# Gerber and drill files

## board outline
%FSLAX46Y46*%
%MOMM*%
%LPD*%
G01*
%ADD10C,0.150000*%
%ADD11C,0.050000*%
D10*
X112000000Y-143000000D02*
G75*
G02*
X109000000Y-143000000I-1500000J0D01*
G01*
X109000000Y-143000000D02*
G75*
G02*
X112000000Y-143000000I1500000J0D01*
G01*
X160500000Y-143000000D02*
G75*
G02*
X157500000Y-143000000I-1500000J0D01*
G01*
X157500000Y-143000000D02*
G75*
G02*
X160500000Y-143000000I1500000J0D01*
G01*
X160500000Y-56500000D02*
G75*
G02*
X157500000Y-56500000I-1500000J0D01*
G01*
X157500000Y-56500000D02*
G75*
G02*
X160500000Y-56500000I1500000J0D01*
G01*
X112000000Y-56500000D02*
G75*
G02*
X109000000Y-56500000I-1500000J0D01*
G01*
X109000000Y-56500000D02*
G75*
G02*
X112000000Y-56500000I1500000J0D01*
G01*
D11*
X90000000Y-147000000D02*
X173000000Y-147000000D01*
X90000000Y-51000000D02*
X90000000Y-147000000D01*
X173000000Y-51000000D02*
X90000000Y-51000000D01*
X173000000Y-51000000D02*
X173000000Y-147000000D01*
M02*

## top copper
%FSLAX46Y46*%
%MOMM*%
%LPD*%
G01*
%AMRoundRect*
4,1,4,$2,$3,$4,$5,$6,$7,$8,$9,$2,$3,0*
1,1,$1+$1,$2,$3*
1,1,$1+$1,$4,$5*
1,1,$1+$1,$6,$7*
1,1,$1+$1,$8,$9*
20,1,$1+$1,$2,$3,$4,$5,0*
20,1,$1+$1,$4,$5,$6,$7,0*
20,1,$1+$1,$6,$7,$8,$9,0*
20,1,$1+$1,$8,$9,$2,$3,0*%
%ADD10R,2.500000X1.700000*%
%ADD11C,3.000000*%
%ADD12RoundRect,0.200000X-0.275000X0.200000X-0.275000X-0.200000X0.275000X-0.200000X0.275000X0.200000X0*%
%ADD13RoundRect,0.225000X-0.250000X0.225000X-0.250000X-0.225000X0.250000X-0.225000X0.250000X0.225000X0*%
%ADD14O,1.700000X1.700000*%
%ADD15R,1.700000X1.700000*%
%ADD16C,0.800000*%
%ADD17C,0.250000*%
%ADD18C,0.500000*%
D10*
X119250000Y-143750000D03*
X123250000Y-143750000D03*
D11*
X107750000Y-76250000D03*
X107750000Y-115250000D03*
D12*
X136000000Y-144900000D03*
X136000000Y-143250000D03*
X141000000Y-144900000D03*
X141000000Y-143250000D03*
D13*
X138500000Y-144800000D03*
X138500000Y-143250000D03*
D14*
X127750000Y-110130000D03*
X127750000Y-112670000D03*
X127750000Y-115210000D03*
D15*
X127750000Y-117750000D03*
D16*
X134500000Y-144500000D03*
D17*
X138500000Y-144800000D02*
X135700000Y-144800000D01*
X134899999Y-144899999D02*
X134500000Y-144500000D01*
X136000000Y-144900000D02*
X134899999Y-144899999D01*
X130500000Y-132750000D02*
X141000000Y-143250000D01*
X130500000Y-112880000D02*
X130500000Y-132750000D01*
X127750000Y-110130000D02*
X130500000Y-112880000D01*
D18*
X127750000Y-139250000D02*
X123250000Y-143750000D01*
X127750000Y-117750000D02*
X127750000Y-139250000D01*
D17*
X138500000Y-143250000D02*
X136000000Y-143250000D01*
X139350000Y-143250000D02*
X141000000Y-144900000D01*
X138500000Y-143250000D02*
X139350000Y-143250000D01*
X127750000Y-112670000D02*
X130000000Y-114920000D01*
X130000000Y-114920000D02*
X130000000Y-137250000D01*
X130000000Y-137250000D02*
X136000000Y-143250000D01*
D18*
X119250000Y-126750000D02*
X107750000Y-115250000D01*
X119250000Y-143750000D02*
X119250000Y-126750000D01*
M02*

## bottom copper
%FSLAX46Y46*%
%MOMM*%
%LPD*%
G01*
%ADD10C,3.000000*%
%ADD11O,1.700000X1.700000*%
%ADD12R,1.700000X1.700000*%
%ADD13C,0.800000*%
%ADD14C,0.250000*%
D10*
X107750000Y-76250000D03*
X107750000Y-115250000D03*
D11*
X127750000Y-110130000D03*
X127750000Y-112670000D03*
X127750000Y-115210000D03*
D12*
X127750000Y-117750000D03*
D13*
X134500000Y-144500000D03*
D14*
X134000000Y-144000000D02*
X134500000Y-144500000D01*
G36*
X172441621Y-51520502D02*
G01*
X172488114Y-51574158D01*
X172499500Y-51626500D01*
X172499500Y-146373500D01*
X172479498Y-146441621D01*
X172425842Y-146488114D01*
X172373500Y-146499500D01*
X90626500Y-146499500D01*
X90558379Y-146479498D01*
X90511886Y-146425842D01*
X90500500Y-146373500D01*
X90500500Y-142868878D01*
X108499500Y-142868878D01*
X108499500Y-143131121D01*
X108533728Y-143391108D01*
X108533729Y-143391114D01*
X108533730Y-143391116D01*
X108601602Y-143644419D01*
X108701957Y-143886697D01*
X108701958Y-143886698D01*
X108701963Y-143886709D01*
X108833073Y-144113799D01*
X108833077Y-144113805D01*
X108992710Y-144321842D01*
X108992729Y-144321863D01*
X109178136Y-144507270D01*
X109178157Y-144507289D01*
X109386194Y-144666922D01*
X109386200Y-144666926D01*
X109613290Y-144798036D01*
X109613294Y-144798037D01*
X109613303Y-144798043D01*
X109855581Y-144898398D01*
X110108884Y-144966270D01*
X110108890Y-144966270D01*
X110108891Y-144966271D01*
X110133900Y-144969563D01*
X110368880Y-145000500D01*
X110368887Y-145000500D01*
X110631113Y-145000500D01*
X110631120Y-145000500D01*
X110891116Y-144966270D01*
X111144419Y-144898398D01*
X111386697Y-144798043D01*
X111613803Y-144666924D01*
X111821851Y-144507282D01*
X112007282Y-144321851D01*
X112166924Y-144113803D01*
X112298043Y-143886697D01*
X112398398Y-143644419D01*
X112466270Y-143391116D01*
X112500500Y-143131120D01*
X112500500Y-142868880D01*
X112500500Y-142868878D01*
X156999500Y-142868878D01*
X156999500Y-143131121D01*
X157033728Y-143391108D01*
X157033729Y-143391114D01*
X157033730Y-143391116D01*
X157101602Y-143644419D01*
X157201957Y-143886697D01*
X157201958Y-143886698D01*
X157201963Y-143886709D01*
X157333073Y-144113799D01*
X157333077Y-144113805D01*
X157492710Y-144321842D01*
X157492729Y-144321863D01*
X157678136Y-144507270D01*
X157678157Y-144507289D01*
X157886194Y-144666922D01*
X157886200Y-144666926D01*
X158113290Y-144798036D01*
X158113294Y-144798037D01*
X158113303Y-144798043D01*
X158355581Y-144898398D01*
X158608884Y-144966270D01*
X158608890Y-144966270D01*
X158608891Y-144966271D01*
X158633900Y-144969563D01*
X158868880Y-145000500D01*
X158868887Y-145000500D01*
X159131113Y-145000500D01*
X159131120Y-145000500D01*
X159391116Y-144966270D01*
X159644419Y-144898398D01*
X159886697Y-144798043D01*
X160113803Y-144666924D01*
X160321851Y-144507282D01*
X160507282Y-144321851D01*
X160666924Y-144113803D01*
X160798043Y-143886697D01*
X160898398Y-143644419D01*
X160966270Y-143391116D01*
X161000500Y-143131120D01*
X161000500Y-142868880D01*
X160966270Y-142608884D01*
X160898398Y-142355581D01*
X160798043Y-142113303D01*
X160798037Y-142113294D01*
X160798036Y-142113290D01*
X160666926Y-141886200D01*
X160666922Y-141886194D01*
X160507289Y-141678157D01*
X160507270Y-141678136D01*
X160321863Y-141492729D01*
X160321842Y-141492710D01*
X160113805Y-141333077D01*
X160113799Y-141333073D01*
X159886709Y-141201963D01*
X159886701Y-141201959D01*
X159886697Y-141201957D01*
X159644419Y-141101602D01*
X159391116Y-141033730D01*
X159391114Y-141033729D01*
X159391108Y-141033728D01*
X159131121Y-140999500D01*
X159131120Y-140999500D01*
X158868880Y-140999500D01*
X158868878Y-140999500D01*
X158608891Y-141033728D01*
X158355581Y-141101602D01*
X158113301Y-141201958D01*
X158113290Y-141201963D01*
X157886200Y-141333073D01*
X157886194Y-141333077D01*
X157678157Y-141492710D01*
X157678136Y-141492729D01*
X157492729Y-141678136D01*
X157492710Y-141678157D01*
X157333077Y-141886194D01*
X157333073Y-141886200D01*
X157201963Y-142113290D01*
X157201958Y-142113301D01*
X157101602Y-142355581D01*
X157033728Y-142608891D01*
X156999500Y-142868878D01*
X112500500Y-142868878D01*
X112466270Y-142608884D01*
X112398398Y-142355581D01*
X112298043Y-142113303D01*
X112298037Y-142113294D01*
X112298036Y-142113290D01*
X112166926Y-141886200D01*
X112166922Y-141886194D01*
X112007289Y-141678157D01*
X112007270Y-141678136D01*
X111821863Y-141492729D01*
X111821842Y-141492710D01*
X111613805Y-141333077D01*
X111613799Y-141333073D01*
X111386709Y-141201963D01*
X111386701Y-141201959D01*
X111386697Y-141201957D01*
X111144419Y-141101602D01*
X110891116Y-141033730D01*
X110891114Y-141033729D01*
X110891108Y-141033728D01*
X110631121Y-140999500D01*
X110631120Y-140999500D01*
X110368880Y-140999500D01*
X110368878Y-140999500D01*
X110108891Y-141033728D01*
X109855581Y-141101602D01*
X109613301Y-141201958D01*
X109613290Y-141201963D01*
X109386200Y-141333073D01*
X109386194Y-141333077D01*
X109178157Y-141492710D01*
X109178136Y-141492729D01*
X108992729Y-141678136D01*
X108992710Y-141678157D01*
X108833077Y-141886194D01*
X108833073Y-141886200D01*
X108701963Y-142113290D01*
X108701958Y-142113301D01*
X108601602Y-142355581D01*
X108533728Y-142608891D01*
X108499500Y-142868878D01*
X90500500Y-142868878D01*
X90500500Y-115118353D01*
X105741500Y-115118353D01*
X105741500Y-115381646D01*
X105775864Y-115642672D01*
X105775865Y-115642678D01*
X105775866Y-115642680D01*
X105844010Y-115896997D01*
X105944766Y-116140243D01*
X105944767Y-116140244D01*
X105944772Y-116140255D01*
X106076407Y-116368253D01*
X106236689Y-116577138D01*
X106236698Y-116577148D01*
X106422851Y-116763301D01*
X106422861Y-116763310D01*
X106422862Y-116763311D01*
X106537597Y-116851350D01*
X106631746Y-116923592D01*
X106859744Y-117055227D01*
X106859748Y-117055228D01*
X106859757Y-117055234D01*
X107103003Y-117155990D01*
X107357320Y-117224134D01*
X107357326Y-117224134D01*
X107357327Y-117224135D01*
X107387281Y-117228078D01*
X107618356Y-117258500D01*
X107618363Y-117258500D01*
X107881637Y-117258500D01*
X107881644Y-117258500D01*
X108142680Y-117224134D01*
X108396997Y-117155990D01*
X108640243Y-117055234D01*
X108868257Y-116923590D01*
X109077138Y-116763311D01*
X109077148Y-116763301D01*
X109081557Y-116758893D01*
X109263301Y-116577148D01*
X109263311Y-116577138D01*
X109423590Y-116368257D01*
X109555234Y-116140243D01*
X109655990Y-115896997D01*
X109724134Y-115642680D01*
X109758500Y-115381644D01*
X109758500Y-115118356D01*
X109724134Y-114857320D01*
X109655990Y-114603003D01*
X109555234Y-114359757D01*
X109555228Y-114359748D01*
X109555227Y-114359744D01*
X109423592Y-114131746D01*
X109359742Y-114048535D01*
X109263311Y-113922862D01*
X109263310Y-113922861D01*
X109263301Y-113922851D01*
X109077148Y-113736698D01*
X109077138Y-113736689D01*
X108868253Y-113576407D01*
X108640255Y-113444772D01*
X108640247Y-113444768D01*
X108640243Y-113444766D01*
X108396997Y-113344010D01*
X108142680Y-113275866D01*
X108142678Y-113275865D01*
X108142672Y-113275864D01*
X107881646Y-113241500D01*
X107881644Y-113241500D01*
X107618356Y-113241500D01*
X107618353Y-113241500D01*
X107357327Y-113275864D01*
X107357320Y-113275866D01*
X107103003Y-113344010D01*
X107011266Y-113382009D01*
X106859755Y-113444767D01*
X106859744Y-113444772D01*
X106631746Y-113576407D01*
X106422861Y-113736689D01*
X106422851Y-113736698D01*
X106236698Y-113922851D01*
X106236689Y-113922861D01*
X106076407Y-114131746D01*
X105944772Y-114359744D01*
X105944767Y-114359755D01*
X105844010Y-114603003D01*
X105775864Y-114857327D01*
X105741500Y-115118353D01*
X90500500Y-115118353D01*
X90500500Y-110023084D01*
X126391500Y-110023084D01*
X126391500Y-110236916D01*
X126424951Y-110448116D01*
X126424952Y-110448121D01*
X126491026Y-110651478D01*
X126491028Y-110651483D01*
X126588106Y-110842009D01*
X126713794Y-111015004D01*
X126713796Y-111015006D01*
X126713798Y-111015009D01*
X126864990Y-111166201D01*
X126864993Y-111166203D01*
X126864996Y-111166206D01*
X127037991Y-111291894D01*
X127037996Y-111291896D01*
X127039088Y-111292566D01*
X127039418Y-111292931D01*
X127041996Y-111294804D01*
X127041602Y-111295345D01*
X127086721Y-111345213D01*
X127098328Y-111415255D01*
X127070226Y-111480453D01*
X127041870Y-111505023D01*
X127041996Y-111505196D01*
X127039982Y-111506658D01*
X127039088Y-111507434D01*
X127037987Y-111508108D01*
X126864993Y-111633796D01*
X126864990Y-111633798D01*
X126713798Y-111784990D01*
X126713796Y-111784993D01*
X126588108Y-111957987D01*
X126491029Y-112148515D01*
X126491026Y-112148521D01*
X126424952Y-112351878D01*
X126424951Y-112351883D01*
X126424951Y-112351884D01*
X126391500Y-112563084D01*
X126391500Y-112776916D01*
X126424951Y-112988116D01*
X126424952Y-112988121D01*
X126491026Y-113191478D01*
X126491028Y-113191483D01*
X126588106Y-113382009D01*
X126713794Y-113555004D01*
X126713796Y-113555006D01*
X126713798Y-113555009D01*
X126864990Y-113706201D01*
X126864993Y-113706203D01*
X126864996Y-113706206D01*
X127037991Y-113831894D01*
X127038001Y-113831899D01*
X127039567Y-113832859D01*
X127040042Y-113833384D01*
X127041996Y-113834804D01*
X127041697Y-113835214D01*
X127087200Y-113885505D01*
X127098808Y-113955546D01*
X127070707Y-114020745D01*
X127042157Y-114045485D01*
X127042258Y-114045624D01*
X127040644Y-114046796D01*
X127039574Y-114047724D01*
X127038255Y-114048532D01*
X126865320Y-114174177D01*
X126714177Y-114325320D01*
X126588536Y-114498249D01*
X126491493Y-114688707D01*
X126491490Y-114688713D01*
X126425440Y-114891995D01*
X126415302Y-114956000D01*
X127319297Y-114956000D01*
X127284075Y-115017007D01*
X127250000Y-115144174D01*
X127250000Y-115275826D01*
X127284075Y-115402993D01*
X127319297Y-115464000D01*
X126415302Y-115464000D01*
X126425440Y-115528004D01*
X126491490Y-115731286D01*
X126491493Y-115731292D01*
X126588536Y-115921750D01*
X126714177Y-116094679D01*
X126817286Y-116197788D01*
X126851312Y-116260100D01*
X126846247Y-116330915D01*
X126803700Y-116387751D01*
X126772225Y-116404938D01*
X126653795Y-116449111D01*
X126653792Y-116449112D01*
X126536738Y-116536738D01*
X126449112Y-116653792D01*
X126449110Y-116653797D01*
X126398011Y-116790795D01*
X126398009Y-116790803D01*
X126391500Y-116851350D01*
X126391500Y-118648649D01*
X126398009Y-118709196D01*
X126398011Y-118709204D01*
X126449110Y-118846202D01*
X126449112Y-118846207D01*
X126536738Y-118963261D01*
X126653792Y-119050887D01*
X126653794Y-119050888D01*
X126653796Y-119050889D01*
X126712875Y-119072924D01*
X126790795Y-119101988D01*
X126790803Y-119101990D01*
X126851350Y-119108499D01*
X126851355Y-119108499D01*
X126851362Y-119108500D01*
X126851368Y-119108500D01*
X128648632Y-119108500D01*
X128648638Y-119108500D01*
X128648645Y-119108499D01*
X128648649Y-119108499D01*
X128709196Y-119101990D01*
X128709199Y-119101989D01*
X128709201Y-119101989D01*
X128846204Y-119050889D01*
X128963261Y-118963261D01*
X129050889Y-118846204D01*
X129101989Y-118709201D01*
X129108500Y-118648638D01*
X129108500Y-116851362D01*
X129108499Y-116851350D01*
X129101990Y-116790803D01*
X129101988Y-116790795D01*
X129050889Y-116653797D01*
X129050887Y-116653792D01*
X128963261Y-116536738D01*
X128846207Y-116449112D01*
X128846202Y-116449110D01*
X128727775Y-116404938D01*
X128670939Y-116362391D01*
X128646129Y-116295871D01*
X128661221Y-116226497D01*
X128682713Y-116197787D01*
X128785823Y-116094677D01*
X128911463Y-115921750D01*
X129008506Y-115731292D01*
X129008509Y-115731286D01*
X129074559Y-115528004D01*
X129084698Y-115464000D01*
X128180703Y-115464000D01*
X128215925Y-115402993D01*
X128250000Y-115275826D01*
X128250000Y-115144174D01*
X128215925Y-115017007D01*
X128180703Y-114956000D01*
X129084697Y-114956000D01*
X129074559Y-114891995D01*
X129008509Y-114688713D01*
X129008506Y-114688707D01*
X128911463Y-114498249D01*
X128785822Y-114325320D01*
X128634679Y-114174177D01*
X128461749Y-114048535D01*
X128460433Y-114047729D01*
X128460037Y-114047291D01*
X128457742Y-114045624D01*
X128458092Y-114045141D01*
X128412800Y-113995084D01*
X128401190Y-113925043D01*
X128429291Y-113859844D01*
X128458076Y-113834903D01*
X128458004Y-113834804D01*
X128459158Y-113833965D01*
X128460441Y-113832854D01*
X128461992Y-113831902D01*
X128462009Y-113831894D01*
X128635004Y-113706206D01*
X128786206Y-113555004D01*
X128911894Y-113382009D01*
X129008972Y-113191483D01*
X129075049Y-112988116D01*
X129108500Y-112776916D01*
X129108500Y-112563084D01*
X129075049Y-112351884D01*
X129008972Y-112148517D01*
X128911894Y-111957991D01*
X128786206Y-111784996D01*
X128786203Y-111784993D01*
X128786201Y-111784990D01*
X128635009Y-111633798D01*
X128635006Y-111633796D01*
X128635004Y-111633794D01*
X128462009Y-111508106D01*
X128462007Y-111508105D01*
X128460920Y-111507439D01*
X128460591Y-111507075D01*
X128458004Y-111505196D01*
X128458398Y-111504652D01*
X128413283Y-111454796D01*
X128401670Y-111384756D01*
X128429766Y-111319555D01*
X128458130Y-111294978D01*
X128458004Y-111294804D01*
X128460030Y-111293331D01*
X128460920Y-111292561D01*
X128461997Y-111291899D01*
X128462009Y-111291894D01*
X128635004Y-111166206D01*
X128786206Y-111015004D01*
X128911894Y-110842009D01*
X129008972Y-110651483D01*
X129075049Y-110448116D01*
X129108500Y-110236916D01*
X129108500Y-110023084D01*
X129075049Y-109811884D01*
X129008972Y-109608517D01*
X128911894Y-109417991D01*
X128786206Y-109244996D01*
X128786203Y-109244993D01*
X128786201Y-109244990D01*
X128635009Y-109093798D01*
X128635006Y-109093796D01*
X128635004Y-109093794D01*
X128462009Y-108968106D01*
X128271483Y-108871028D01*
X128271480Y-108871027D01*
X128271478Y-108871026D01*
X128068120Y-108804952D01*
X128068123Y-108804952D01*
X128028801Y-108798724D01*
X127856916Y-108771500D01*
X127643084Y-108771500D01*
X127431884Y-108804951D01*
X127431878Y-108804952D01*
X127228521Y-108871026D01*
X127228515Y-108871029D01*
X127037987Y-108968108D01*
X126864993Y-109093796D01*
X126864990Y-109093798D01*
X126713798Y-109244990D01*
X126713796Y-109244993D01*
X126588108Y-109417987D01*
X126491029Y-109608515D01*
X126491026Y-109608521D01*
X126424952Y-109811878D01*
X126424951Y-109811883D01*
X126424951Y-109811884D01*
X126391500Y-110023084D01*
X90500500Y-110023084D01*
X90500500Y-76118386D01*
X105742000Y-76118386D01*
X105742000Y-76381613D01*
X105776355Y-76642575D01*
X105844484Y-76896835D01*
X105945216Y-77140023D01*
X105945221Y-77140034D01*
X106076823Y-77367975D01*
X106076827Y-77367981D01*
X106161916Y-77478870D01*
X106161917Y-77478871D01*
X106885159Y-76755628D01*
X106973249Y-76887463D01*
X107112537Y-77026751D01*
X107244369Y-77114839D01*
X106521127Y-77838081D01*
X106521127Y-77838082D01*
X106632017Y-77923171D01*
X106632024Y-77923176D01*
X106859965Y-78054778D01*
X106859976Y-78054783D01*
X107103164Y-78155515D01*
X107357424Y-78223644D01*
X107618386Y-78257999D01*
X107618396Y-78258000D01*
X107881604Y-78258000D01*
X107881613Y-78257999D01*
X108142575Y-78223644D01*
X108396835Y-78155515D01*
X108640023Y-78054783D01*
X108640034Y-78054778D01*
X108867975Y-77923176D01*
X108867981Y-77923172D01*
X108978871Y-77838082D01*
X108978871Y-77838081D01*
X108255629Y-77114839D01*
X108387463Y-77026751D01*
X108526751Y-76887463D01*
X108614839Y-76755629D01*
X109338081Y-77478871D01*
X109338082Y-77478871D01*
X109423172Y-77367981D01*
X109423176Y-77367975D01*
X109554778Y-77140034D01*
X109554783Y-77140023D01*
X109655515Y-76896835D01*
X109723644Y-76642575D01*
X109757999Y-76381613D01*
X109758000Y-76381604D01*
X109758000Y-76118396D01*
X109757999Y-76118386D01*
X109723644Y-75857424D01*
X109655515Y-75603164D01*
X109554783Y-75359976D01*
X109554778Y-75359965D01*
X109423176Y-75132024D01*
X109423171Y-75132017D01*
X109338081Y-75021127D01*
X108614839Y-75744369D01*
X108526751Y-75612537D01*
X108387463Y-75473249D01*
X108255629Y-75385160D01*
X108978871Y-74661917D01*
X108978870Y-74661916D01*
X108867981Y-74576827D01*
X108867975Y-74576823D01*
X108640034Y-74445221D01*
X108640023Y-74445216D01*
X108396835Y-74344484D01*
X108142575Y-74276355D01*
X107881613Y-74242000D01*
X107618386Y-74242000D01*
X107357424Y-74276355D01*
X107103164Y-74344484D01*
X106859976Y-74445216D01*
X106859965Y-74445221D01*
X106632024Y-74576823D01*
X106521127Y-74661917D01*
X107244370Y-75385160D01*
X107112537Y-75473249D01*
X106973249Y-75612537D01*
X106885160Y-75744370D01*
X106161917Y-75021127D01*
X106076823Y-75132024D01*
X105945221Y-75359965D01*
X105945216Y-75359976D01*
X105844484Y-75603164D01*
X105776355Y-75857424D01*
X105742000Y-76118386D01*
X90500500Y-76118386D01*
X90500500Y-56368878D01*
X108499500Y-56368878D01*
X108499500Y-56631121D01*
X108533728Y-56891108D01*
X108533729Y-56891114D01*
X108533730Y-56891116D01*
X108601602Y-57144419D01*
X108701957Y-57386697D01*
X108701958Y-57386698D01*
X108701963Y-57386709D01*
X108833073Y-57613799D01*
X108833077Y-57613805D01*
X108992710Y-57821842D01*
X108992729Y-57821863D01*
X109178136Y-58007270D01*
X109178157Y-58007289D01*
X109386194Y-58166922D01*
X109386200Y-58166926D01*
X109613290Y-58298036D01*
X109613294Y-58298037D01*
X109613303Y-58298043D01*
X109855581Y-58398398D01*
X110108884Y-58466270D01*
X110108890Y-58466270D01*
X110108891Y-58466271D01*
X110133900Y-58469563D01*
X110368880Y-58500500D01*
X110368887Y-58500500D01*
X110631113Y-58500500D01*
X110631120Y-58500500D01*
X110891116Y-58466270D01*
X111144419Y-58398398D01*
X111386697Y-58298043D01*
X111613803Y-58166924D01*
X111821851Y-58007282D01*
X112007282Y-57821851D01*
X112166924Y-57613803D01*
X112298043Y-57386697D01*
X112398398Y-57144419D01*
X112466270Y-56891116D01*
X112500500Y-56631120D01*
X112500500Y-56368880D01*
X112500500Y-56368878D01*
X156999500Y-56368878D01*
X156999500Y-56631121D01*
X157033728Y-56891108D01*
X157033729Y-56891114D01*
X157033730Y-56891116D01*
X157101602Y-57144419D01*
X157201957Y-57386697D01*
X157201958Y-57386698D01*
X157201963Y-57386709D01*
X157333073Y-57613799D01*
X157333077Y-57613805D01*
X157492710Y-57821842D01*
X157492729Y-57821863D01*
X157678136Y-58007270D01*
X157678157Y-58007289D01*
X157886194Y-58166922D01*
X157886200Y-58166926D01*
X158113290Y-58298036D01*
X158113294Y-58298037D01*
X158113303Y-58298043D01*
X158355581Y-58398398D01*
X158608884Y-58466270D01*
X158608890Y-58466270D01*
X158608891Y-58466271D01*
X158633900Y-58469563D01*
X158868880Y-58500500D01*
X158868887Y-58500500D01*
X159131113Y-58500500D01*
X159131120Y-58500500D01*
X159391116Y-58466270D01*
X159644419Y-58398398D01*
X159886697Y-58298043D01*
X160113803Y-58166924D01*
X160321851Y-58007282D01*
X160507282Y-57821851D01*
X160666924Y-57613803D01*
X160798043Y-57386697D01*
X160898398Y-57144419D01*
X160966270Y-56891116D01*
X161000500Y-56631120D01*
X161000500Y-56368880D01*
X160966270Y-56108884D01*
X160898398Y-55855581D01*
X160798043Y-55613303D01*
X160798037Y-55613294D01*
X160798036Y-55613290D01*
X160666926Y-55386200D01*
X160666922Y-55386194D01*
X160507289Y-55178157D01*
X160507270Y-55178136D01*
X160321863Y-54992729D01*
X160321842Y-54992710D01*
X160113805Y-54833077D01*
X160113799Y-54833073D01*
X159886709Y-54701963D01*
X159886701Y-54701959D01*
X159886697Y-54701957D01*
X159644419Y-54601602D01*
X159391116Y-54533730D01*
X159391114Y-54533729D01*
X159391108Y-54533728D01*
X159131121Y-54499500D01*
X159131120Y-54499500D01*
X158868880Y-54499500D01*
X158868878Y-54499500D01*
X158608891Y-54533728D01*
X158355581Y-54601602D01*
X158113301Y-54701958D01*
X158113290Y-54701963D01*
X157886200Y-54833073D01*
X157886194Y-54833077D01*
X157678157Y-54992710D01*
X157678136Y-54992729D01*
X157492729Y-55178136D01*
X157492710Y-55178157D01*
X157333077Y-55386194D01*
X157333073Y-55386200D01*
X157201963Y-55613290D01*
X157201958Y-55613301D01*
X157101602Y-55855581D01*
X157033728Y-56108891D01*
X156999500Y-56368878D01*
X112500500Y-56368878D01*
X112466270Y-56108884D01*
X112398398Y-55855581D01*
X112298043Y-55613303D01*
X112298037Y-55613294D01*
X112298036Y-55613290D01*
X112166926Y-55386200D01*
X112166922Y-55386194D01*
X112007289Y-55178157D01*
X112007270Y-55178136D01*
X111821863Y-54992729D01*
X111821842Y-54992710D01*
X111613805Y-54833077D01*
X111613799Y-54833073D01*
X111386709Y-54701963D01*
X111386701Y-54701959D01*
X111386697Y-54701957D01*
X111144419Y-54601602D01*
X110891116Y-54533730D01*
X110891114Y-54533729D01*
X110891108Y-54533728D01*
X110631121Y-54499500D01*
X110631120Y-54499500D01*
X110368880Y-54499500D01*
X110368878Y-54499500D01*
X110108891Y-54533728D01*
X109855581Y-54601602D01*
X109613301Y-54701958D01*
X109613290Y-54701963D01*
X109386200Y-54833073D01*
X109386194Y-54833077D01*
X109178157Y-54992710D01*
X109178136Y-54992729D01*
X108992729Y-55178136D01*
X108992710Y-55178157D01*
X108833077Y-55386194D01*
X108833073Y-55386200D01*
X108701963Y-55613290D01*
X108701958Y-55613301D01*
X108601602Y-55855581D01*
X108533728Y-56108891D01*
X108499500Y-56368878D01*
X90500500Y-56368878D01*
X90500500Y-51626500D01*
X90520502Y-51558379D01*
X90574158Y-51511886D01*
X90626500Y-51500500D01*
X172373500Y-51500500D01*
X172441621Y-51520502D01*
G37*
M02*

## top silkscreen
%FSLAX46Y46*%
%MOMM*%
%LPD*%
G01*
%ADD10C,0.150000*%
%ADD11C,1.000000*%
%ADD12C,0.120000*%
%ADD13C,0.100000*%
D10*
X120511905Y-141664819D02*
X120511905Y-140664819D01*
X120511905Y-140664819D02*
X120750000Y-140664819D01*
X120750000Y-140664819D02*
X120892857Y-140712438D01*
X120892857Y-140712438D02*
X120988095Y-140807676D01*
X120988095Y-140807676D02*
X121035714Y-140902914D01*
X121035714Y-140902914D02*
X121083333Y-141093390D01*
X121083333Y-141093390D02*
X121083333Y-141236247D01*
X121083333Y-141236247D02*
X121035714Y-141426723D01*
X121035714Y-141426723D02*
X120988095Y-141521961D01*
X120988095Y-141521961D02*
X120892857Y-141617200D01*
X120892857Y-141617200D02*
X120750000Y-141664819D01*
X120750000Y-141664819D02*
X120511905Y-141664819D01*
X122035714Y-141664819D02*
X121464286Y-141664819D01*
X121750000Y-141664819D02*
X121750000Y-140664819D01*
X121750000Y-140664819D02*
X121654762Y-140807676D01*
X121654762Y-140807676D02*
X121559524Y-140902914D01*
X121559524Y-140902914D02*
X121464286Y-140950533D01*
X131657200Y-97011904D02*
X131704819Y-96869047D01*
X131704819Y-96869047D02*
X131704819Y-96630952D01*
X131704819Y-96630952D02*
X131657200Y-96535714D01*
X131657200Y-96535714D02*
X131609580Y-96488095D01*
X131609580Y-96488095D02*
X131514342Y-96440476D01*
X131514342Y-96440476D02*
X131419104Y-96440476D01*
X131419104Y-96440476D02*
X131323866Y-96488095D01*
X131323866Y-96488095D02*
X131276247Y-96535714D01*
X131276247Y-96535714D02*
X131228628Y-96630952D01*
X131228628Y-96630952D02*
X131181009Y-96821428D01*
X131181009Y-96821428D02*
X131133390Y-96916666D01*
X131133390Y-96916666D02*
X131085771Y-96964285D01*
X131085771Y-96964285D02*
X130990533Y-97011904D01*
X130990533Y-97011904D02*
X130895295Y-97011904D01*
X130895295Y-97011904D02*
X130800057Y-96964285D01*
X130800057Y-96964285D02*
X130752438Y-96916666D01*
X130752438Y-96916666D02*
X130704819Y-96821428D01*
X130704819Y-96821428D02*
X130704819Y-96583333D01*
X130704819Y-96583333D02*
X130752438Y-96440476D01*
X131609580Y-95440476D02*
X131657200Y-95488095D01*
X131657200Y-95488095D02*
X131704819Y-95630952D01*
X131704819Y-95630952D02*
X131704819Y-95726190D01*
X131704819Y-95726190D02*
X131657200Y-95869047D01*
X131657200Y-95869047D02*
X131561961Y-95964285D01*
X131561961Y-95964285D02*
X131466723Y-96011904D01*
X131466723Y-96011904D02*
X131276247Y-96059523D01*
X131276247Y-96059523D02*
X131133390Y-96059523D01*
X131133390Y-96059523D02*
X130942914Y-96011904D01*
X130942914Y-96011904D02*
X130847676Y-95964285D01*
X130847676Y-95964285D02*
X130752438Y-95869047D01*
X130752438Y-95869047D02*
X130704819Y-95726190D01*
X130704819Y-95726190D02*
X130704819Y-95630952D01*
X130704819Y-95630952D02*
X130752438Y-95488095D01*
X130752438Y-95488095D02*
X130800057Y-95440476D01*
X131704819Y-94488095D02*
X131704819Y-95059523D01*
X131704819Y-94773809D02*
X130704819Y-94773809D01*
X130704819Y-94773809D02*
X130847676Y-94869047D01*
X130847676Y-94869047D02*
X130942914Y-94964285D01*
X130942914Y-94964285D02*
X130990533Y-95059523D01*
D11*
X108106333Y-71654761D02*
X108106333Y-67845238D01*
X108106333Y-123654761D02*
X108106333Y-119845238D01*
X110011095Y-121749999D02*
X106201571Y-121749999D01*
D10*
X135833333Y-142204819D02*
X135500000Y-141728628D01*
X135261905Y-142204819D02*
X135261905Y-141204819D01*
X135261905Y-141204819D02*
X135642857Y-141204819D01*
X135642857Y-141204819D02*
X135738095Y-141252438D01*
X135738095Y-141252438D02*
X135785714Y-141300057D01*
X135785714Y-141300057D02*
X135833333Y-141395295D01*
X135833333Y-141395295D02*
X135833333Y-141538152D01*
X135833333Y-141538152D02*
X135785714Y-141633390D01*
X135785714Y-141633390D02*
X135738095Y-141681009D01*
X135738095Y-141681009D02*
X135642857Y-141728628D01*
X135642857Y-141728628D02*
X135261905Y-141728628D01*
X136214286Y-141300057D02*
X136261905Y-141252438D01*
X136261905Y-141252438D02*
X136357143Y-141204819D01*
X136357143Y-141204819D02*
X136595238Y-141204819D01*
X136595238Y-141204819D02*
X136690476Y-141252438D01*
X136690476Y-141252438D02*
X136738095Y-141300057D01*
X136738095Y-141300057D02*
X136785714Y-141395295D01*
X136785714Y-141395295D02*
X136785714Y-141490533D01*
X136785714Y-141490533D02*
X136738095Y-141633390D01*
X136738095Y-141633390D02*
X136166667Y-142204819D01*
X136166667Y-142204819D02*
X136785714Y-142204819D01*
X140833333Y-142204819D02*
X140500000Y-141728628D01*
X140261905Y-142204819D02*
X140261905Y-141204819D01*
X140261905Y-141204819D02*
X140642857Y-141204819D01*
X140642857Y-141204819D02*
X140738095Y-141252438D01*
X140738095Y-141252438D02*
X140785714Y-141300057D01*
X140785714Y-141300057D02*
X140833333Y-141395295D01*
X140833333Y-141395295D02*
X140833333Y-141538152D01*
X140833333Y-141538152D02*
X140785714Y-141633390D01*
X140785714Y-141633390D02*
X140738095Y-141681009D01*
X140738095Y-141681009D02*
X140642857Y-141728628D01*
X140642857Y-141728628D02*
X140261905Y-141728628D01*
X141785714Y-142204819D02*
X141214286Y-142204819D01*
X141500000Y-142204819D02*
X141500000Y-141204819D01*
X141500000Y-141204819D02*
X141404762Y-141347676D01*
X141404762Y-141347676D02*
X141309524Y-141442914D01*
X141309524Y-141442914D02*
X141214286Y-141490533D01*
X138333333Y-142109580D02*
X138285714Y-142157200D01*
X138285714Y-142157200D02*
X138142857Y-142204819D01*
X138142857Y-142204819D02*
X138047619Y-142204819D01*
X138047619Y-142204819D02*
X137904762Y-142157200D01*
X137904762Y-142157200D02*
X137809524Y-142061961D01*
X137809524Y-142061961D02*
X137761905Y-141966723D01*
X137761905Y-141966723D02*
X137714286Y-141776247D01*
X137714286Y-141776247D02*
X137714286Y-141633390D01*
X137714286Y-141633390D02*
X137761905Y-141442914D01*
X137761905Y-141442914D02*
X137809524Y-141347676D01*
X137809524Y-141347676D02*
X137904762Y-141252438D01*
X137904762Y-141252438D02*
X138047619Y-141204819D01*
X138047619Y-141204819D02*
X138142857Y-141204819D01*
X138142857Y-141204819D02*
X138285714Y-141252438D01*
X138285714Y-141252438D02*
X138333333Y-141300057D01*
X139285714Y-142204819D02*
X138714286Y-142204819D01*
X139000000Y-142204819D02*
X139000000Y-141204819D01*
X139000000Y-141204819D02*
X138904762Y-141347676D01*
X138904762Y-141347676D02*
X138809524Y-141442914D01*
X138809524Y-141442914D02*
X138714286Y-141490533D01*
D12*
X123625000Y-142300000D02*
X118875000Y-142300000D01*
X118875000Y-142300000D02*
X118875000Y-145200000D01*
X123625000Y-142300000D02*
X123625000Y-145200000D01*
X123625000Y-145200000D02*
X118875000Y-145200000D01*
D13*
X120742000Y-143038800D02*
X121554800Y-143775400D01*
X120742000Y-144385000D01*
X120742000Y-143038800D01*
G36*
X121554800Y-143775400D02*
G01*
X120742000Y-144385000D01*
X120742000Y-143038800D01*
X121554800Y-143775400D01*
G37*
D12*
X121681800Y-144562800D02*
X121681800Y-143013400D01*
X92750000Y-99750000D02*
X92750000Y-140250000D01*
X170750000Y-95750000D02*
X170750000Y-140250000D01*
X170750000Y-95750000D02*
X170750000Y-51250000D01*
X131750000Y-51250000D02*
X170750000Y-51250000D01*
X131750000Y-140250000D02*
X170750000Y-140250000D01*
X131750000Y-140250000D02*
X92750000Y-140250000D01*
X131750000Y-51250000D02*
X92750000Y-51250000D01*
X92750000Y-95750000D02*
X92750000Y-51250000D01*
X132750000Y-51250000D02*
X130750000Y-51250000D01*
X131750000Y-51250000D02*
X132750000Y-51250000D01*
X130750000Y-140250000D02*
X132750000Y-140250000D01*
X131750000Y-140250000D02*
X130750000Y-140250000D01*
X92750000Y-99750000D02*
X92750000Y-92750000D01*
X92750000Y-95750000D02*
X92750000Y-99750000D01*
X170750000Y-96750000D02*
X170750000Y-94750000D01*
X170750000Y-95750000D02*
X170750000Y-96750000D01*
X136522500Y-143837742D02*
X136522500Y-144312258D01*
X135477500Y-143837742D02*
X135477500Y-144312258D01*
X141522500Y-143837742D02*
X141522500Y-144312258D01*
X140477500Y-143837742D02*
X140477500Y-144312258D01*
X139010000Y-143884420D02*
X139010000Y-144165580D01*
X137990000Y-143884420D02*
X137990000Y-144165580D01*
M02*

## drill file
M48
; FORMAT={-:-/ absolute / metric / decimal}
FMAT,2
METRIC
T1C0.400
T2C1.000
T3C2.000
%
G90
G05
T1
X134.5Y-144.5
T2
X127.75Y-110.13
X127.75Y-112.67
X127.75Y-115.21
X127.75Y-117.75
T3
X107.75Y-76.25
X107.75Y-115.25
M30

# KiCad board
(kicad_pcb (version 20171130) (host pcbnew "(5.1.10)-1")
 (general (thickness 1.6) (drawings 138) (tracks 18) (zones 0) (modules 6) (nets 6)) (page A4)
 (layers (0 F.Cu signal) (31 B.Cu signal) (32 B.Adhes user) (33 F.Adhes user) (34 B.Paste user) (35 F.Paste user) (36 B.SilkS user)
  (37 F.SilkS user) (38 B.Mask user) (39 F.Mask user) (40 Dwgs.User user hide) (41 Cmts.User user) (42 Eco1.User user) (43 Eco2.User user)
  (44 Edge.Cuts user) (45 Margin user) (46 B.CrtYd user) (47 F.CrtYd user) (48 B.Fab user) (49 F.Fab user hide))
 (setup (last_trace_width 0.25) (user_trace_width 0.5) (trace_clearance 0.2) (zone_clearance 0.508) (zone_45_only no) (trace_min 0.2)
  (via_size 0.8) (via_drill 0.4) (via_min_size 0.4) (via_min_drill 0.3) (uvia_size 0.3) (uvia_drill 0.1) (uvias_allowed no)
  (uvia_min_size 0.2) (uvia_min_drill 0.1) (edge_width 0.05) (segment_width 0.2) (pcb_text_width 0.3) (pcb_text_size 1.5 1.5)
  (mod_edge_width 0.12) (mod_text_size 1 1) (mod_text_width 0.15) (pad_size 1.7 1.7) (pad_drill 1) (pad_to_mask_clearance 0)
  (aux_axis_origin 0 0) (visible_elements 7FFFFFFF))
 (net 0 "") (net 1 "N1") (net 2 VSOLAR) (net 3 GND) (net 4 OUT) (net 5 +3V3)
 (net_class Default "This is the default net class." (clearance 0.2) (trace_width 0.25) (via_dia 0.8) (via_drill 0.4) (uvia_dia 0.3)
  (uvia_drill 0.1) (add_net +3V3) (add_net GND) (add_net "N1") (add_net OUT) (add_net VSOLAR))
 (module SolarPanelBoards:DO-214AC (layer F.Cu) (at 121.25 143.75 180)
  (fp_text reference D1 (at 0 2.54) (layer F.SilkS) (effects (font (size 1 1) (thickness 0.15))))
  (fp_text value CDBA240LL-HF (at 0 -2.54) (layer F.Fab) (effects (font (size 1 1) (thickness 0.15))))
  (fp_line (start -2.375 1.45) (end 2.375 1.45) (layer F.SilkS) (width 0.12))
  (fp_line (start 2.375 1.45) (end 2.375 -1.45) (layer F.SilkS) (width 0.12))
  (fp_line (start -2.375 1.45) (end -2.375 -1.45) (layer F.SilkS) (width 0.12))
  (fp_line (start -2.375 -1.45) (end 2.375 -1.45) (layer F.SilkS) (width 0.12))
  (fp_poly (pts (xy 0.508 0.7112) (xy -0.3048 -0.0254) (xy 0.508 -0.635)) (layer F.SilkS) (width 0.1))
  (fp_line (start -0.4318 -0.8128) (end -0.4318 0.7366) (layer F.SilkS) (width 0.12))
  (pad 2 smd rect (at 2 0 180) (size 2.5 1.7) (layers F.Cu F.Paste F.Mask) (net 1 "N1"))
  (pad 1 smd rect (at -2 0 180) (size 2.5 1.7) (layers F.Cu F.Paste F.Mask) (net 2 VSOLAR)))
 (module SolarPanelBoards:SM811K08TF (layer F.Cu) (at 131.75 95.75 270)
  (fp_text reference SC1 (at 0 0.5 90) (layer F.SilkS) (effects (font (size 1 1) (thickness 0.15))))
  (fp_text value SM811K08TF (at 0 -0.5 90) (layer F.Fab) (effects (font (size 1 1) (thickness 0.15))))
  (fp_line (start 4 39) (end 44.5 39) (layer F.SilkS) (width 0.12))
  (fp_line (start 0 -39) (end 44.5 -39) (layer F.SilkS) (width 0.12))
  (fp_line (start 0 -39) (end -44.5 -39) (layer F.SilkS) (width 0.12))
  (fp_line (start -44.5 0) (end -44.5 -39) (layer F.SilkS) (width 0.12))
  (fp_line (start 44.5 0) (end 44.5 -39) (layer F.SilkS) (width 0.12))
  (fp_line (start 44.5 0) (end 44.5 39) (layer F.SilkS) (width 0.12))
  (fp_line (start -44.5 0) (end -44.5 39) (layer F.SilkS) (width 0.12))
  (fp_line (start 0 39) (end -44.5 39) (layer F.SilkS) (width 0.12))
  (fp_line (start -44.5 -1) (end -44.5 1) (layer F.SilkS) (width 0.12))
  (fp_line (start -44.5 0) (end -44.5 -1) (layer F.SilkS) (width 0.12))
  (fp_line (start 44.5 1) (end 44.5 -1) (layer F.SilkS) (width 0.12))
  (fp_line (start 44.5 0) (end 44.5 1) (layer F.SilkS) (width 0.12))
  (fp_line (start 4 39) (end -3 39) (layer F.SilkS) (width 0.12))
  (fp_line (start 0 39) (end 4 39) (layer F.SilkS) (width 0.12))
  (fp_line (start 1 -39) (end -1 -39) (layer F.SilkS) (width 0.12))
  (fp_line (start 0 -39) (end 1 -39) (layer F.SilkS) (width 0.12))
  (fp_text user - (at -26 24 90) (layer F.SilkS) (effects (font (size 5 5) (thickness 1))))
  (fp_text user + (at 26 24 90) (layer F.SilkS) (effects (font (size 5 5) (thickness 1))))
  (pad 2 thru_hole circle (at -19.5 24 270) (size 3 3) (drill 2) (layers *.Cu *.Mask) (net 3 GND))
  (pad 1 thru_hole circle (at 19.5 24 270) (size 3 3) (drill 2) (layers *.Cu *.Mask) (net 1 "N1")))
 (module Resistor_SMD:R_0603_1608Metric (layer F.Cu) (at 136 144.075 270)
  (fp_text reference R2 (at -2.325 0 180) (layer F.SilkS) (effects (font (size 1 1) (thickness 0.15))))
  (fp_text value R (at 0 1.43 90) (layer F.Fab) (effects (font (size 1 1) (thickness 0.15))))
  (fp_line (start -0.237258 -0.5225) (end 0.237258 -0.5225) (layer F.SilkS) (width 0.12))
  (fp_line (start -0.237258 0.5225) (end 0.237258 0.5225) (layer F.SilkS) (width 0.12))
  (pad 2 smd roundrect (at 0.825 0 270) (size 0.8 0.95) (layers F.Cu F.Paste F.Mask) (roundrect_rratio 0.25) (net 3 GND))
  (pad 1 smd roundrect (at -0.825 0 270) (size 0.8 0.95) (layers F.Cu F.Paste F.Mask) (roundrect_rratio 0.25) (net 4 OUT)))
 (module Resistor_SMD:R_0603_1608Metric (layer F.Cu) (at 141 144.075 270)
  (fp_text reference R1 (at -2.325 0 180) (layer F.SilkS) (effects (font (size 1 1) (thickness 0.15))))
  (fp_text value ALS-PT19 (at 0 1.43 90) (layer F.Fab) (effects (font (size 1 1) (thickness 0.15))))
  (fp_line (start -0.237258 -0.5225) (end 0.237258 -0.5225) (layer F.SilkS) (width 0.12))
  (fp_line (start -0.237258 0.5225) (end 0.237258 0.5225) (layer F.SilkS) (width 0.12))
  (pad 2 smd roundrect (at 0.825 0 270) (size 0.8 0.95) (layers F.Cu F.Paste F.Mask) (roundrect_rratio 0.25) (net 4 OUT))
  (pad 1 smd roundrect (at -0.825 0 270) (size 0.8 0.95) (layers F.Cu F.Paste F.Mask) (roundrect_rratio 0.25) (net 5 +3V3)))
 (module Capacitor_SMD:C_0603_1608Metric (layer F.Cu) (at 138.5 144.025 270)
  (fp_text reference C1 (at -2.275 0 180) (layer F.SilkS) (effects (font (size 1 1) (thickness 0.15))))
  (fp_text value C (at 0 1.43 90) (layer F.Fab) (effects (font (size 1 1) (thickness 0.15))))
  (fp_line (start -0.14058 -0.51) (end 0.14058 -0.51) (layer F.SilkS) (width 0.12))
  (fp_line (start -0.14058 0.51) (end 0.14058 0.51) (layer F.SilkS) (width 0.12))
  (pad 2 smd roundrect (at 0.775 0 270) (size 0.9 0.95) (layers F.Cu F.Paste F.Mask) (roundrect_rratio 0.25) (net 3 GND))
  (pad 1 smd roundrect (at -0.775 0 270) (size 0.9 0.95) (layers F.Cu F.Paste F.Mask) (roundrect_rratio 0.25) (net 4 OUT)))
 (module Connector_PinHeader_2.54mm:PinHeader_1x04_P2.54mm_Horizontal (layer B.Cu) (at 127.75 117.75)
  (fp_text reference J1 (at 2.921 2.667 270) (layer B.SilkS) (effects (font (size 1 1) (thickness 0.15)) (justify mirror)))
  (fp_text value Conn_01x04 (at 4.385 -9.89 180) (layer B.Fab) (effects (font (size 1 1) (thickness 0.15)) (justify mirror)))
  (pad 4 thru_hole oval (at 0 -7.62) (size 1.7 1.7) (drill 1) (layers *.Cu *.Mask) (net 5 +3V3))
  (pad 3 thru_hole oval (at 0 -5.08) (size 1.7 1.7) (drill 1) (layers *.Cu *.Mask) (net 4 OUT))
  (pad 2 thru_hole oval (at 0 -2.54) (size 1.7 1.7) (drill 1) (layers *.Cu *.Mask) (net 3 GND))
  (pad 1 thru_hole rect (at 0 0) (size 1.7 1.7) (drill 1) (layers *.Cu *.Mask) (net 2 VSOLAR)))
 (gr_circle (center 110.5 143) (end 112 143) (layer Edge.Cuts) (width 0.15))
 (gr_circle (center 159 143) (end 160.5 143) (layer Edge.Cuts) (width 0.15))
 (gr_circle (center 159 56.5) (end 160.5 56.5) (layer Edge.Cuts) (width 0.15))
 (gr_circle (center 110.5 56.5) (end 112 56.5) (layer Edge.Cuts) (width 0.15))
 (gr_line (start 90 147) (end 173 147) (layer Edge.Cuts) (width 0.05))
 (gr_line (start 90 51) (end 90 147) (layer Edge.Cuts) (width 0.05))
 (gr_line (start 173 51) (end 90 51) (layer Edge.Cuts) (width 0.05))
 (gr_line (start 173 51) (end 173 147) (layer Edge.Cuts) (width 0.05))
 (segment (start 138.5 144.8) (end 135.7 144.8) (width 0.25) (layer F.Cu) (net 3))
 (via (at 134.5 144.5) (size 0.8) (drill 0.4) (layers F.Cu B.Cu) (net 3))
 (segment (start 134.899999 144.899999) (end 134.5 144.5) (width 0.25) (layer F.Cu) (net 3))
 (segment (start 136 144.9) (end 134.899999 144.899999) (width 0.25) (layer F.Cu) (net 3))
 (segment (start 134 144) (end 134.5 144.5) (width 0.25) (layer B.Cu) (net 3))
 (segment (start 130.5 132.75) (end 141 143.25) (width 0.25) (layer F.Cu) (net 5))
 (segment (start 130.5 112.88) (end 130.5 132.75) (width 0.25) (layer F.Cu) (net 5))
 (segment (start 127.75 110.13) (end 130.5 112.88) (width 0.25) (layer F.Cu) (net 5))
 (segment (start 127.75 139.25) (end 123.25 143.75) (width 0.5) (layer F.Cu) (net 2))
 (segment (start 127.75 117.75) (end 127.75 139.25) (width 0.5) (layer F.Cu) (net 2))
 (segment (start 138.5 143.25) (end 136 143.25) (width 0.25) (layer F.Cu) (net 4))
 (segment (start 139.35 143.25) (end 141 144.9) (width 0.25) (layer F.Cu) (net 4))
 (segment (start 138.5 143.25) (end 139.35 143.25) (width 0.25) (layer F.Cu) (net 4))
 (segment (start 127.75 112.67) (end 130 114.92) (width 0.25) (layer F.Cu) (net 4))
 (segment (start 130 114.92) (end 130 137.25) (width 0.25) (layer F.Cu) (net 4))
 (segment (start 130 137.25) (end 136 143.25) (width 0.25) (layer F.Cu) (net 4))
 (segment (start 119.25 126.75) (end 107.75 115.25) (width 0.5) (layer F.Cu) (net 1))
 (segment (start 119.25 143.75) (end 119.25 126.75) (width 0.5) (layer F.Cu) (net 1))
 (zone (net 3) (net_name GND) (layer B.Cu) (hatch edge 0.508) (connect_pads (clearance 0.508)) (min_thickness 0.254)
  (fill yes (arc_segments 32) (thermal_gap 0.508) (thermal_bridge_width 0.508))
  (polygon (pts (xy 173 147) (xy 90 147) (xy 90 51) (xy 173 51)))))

